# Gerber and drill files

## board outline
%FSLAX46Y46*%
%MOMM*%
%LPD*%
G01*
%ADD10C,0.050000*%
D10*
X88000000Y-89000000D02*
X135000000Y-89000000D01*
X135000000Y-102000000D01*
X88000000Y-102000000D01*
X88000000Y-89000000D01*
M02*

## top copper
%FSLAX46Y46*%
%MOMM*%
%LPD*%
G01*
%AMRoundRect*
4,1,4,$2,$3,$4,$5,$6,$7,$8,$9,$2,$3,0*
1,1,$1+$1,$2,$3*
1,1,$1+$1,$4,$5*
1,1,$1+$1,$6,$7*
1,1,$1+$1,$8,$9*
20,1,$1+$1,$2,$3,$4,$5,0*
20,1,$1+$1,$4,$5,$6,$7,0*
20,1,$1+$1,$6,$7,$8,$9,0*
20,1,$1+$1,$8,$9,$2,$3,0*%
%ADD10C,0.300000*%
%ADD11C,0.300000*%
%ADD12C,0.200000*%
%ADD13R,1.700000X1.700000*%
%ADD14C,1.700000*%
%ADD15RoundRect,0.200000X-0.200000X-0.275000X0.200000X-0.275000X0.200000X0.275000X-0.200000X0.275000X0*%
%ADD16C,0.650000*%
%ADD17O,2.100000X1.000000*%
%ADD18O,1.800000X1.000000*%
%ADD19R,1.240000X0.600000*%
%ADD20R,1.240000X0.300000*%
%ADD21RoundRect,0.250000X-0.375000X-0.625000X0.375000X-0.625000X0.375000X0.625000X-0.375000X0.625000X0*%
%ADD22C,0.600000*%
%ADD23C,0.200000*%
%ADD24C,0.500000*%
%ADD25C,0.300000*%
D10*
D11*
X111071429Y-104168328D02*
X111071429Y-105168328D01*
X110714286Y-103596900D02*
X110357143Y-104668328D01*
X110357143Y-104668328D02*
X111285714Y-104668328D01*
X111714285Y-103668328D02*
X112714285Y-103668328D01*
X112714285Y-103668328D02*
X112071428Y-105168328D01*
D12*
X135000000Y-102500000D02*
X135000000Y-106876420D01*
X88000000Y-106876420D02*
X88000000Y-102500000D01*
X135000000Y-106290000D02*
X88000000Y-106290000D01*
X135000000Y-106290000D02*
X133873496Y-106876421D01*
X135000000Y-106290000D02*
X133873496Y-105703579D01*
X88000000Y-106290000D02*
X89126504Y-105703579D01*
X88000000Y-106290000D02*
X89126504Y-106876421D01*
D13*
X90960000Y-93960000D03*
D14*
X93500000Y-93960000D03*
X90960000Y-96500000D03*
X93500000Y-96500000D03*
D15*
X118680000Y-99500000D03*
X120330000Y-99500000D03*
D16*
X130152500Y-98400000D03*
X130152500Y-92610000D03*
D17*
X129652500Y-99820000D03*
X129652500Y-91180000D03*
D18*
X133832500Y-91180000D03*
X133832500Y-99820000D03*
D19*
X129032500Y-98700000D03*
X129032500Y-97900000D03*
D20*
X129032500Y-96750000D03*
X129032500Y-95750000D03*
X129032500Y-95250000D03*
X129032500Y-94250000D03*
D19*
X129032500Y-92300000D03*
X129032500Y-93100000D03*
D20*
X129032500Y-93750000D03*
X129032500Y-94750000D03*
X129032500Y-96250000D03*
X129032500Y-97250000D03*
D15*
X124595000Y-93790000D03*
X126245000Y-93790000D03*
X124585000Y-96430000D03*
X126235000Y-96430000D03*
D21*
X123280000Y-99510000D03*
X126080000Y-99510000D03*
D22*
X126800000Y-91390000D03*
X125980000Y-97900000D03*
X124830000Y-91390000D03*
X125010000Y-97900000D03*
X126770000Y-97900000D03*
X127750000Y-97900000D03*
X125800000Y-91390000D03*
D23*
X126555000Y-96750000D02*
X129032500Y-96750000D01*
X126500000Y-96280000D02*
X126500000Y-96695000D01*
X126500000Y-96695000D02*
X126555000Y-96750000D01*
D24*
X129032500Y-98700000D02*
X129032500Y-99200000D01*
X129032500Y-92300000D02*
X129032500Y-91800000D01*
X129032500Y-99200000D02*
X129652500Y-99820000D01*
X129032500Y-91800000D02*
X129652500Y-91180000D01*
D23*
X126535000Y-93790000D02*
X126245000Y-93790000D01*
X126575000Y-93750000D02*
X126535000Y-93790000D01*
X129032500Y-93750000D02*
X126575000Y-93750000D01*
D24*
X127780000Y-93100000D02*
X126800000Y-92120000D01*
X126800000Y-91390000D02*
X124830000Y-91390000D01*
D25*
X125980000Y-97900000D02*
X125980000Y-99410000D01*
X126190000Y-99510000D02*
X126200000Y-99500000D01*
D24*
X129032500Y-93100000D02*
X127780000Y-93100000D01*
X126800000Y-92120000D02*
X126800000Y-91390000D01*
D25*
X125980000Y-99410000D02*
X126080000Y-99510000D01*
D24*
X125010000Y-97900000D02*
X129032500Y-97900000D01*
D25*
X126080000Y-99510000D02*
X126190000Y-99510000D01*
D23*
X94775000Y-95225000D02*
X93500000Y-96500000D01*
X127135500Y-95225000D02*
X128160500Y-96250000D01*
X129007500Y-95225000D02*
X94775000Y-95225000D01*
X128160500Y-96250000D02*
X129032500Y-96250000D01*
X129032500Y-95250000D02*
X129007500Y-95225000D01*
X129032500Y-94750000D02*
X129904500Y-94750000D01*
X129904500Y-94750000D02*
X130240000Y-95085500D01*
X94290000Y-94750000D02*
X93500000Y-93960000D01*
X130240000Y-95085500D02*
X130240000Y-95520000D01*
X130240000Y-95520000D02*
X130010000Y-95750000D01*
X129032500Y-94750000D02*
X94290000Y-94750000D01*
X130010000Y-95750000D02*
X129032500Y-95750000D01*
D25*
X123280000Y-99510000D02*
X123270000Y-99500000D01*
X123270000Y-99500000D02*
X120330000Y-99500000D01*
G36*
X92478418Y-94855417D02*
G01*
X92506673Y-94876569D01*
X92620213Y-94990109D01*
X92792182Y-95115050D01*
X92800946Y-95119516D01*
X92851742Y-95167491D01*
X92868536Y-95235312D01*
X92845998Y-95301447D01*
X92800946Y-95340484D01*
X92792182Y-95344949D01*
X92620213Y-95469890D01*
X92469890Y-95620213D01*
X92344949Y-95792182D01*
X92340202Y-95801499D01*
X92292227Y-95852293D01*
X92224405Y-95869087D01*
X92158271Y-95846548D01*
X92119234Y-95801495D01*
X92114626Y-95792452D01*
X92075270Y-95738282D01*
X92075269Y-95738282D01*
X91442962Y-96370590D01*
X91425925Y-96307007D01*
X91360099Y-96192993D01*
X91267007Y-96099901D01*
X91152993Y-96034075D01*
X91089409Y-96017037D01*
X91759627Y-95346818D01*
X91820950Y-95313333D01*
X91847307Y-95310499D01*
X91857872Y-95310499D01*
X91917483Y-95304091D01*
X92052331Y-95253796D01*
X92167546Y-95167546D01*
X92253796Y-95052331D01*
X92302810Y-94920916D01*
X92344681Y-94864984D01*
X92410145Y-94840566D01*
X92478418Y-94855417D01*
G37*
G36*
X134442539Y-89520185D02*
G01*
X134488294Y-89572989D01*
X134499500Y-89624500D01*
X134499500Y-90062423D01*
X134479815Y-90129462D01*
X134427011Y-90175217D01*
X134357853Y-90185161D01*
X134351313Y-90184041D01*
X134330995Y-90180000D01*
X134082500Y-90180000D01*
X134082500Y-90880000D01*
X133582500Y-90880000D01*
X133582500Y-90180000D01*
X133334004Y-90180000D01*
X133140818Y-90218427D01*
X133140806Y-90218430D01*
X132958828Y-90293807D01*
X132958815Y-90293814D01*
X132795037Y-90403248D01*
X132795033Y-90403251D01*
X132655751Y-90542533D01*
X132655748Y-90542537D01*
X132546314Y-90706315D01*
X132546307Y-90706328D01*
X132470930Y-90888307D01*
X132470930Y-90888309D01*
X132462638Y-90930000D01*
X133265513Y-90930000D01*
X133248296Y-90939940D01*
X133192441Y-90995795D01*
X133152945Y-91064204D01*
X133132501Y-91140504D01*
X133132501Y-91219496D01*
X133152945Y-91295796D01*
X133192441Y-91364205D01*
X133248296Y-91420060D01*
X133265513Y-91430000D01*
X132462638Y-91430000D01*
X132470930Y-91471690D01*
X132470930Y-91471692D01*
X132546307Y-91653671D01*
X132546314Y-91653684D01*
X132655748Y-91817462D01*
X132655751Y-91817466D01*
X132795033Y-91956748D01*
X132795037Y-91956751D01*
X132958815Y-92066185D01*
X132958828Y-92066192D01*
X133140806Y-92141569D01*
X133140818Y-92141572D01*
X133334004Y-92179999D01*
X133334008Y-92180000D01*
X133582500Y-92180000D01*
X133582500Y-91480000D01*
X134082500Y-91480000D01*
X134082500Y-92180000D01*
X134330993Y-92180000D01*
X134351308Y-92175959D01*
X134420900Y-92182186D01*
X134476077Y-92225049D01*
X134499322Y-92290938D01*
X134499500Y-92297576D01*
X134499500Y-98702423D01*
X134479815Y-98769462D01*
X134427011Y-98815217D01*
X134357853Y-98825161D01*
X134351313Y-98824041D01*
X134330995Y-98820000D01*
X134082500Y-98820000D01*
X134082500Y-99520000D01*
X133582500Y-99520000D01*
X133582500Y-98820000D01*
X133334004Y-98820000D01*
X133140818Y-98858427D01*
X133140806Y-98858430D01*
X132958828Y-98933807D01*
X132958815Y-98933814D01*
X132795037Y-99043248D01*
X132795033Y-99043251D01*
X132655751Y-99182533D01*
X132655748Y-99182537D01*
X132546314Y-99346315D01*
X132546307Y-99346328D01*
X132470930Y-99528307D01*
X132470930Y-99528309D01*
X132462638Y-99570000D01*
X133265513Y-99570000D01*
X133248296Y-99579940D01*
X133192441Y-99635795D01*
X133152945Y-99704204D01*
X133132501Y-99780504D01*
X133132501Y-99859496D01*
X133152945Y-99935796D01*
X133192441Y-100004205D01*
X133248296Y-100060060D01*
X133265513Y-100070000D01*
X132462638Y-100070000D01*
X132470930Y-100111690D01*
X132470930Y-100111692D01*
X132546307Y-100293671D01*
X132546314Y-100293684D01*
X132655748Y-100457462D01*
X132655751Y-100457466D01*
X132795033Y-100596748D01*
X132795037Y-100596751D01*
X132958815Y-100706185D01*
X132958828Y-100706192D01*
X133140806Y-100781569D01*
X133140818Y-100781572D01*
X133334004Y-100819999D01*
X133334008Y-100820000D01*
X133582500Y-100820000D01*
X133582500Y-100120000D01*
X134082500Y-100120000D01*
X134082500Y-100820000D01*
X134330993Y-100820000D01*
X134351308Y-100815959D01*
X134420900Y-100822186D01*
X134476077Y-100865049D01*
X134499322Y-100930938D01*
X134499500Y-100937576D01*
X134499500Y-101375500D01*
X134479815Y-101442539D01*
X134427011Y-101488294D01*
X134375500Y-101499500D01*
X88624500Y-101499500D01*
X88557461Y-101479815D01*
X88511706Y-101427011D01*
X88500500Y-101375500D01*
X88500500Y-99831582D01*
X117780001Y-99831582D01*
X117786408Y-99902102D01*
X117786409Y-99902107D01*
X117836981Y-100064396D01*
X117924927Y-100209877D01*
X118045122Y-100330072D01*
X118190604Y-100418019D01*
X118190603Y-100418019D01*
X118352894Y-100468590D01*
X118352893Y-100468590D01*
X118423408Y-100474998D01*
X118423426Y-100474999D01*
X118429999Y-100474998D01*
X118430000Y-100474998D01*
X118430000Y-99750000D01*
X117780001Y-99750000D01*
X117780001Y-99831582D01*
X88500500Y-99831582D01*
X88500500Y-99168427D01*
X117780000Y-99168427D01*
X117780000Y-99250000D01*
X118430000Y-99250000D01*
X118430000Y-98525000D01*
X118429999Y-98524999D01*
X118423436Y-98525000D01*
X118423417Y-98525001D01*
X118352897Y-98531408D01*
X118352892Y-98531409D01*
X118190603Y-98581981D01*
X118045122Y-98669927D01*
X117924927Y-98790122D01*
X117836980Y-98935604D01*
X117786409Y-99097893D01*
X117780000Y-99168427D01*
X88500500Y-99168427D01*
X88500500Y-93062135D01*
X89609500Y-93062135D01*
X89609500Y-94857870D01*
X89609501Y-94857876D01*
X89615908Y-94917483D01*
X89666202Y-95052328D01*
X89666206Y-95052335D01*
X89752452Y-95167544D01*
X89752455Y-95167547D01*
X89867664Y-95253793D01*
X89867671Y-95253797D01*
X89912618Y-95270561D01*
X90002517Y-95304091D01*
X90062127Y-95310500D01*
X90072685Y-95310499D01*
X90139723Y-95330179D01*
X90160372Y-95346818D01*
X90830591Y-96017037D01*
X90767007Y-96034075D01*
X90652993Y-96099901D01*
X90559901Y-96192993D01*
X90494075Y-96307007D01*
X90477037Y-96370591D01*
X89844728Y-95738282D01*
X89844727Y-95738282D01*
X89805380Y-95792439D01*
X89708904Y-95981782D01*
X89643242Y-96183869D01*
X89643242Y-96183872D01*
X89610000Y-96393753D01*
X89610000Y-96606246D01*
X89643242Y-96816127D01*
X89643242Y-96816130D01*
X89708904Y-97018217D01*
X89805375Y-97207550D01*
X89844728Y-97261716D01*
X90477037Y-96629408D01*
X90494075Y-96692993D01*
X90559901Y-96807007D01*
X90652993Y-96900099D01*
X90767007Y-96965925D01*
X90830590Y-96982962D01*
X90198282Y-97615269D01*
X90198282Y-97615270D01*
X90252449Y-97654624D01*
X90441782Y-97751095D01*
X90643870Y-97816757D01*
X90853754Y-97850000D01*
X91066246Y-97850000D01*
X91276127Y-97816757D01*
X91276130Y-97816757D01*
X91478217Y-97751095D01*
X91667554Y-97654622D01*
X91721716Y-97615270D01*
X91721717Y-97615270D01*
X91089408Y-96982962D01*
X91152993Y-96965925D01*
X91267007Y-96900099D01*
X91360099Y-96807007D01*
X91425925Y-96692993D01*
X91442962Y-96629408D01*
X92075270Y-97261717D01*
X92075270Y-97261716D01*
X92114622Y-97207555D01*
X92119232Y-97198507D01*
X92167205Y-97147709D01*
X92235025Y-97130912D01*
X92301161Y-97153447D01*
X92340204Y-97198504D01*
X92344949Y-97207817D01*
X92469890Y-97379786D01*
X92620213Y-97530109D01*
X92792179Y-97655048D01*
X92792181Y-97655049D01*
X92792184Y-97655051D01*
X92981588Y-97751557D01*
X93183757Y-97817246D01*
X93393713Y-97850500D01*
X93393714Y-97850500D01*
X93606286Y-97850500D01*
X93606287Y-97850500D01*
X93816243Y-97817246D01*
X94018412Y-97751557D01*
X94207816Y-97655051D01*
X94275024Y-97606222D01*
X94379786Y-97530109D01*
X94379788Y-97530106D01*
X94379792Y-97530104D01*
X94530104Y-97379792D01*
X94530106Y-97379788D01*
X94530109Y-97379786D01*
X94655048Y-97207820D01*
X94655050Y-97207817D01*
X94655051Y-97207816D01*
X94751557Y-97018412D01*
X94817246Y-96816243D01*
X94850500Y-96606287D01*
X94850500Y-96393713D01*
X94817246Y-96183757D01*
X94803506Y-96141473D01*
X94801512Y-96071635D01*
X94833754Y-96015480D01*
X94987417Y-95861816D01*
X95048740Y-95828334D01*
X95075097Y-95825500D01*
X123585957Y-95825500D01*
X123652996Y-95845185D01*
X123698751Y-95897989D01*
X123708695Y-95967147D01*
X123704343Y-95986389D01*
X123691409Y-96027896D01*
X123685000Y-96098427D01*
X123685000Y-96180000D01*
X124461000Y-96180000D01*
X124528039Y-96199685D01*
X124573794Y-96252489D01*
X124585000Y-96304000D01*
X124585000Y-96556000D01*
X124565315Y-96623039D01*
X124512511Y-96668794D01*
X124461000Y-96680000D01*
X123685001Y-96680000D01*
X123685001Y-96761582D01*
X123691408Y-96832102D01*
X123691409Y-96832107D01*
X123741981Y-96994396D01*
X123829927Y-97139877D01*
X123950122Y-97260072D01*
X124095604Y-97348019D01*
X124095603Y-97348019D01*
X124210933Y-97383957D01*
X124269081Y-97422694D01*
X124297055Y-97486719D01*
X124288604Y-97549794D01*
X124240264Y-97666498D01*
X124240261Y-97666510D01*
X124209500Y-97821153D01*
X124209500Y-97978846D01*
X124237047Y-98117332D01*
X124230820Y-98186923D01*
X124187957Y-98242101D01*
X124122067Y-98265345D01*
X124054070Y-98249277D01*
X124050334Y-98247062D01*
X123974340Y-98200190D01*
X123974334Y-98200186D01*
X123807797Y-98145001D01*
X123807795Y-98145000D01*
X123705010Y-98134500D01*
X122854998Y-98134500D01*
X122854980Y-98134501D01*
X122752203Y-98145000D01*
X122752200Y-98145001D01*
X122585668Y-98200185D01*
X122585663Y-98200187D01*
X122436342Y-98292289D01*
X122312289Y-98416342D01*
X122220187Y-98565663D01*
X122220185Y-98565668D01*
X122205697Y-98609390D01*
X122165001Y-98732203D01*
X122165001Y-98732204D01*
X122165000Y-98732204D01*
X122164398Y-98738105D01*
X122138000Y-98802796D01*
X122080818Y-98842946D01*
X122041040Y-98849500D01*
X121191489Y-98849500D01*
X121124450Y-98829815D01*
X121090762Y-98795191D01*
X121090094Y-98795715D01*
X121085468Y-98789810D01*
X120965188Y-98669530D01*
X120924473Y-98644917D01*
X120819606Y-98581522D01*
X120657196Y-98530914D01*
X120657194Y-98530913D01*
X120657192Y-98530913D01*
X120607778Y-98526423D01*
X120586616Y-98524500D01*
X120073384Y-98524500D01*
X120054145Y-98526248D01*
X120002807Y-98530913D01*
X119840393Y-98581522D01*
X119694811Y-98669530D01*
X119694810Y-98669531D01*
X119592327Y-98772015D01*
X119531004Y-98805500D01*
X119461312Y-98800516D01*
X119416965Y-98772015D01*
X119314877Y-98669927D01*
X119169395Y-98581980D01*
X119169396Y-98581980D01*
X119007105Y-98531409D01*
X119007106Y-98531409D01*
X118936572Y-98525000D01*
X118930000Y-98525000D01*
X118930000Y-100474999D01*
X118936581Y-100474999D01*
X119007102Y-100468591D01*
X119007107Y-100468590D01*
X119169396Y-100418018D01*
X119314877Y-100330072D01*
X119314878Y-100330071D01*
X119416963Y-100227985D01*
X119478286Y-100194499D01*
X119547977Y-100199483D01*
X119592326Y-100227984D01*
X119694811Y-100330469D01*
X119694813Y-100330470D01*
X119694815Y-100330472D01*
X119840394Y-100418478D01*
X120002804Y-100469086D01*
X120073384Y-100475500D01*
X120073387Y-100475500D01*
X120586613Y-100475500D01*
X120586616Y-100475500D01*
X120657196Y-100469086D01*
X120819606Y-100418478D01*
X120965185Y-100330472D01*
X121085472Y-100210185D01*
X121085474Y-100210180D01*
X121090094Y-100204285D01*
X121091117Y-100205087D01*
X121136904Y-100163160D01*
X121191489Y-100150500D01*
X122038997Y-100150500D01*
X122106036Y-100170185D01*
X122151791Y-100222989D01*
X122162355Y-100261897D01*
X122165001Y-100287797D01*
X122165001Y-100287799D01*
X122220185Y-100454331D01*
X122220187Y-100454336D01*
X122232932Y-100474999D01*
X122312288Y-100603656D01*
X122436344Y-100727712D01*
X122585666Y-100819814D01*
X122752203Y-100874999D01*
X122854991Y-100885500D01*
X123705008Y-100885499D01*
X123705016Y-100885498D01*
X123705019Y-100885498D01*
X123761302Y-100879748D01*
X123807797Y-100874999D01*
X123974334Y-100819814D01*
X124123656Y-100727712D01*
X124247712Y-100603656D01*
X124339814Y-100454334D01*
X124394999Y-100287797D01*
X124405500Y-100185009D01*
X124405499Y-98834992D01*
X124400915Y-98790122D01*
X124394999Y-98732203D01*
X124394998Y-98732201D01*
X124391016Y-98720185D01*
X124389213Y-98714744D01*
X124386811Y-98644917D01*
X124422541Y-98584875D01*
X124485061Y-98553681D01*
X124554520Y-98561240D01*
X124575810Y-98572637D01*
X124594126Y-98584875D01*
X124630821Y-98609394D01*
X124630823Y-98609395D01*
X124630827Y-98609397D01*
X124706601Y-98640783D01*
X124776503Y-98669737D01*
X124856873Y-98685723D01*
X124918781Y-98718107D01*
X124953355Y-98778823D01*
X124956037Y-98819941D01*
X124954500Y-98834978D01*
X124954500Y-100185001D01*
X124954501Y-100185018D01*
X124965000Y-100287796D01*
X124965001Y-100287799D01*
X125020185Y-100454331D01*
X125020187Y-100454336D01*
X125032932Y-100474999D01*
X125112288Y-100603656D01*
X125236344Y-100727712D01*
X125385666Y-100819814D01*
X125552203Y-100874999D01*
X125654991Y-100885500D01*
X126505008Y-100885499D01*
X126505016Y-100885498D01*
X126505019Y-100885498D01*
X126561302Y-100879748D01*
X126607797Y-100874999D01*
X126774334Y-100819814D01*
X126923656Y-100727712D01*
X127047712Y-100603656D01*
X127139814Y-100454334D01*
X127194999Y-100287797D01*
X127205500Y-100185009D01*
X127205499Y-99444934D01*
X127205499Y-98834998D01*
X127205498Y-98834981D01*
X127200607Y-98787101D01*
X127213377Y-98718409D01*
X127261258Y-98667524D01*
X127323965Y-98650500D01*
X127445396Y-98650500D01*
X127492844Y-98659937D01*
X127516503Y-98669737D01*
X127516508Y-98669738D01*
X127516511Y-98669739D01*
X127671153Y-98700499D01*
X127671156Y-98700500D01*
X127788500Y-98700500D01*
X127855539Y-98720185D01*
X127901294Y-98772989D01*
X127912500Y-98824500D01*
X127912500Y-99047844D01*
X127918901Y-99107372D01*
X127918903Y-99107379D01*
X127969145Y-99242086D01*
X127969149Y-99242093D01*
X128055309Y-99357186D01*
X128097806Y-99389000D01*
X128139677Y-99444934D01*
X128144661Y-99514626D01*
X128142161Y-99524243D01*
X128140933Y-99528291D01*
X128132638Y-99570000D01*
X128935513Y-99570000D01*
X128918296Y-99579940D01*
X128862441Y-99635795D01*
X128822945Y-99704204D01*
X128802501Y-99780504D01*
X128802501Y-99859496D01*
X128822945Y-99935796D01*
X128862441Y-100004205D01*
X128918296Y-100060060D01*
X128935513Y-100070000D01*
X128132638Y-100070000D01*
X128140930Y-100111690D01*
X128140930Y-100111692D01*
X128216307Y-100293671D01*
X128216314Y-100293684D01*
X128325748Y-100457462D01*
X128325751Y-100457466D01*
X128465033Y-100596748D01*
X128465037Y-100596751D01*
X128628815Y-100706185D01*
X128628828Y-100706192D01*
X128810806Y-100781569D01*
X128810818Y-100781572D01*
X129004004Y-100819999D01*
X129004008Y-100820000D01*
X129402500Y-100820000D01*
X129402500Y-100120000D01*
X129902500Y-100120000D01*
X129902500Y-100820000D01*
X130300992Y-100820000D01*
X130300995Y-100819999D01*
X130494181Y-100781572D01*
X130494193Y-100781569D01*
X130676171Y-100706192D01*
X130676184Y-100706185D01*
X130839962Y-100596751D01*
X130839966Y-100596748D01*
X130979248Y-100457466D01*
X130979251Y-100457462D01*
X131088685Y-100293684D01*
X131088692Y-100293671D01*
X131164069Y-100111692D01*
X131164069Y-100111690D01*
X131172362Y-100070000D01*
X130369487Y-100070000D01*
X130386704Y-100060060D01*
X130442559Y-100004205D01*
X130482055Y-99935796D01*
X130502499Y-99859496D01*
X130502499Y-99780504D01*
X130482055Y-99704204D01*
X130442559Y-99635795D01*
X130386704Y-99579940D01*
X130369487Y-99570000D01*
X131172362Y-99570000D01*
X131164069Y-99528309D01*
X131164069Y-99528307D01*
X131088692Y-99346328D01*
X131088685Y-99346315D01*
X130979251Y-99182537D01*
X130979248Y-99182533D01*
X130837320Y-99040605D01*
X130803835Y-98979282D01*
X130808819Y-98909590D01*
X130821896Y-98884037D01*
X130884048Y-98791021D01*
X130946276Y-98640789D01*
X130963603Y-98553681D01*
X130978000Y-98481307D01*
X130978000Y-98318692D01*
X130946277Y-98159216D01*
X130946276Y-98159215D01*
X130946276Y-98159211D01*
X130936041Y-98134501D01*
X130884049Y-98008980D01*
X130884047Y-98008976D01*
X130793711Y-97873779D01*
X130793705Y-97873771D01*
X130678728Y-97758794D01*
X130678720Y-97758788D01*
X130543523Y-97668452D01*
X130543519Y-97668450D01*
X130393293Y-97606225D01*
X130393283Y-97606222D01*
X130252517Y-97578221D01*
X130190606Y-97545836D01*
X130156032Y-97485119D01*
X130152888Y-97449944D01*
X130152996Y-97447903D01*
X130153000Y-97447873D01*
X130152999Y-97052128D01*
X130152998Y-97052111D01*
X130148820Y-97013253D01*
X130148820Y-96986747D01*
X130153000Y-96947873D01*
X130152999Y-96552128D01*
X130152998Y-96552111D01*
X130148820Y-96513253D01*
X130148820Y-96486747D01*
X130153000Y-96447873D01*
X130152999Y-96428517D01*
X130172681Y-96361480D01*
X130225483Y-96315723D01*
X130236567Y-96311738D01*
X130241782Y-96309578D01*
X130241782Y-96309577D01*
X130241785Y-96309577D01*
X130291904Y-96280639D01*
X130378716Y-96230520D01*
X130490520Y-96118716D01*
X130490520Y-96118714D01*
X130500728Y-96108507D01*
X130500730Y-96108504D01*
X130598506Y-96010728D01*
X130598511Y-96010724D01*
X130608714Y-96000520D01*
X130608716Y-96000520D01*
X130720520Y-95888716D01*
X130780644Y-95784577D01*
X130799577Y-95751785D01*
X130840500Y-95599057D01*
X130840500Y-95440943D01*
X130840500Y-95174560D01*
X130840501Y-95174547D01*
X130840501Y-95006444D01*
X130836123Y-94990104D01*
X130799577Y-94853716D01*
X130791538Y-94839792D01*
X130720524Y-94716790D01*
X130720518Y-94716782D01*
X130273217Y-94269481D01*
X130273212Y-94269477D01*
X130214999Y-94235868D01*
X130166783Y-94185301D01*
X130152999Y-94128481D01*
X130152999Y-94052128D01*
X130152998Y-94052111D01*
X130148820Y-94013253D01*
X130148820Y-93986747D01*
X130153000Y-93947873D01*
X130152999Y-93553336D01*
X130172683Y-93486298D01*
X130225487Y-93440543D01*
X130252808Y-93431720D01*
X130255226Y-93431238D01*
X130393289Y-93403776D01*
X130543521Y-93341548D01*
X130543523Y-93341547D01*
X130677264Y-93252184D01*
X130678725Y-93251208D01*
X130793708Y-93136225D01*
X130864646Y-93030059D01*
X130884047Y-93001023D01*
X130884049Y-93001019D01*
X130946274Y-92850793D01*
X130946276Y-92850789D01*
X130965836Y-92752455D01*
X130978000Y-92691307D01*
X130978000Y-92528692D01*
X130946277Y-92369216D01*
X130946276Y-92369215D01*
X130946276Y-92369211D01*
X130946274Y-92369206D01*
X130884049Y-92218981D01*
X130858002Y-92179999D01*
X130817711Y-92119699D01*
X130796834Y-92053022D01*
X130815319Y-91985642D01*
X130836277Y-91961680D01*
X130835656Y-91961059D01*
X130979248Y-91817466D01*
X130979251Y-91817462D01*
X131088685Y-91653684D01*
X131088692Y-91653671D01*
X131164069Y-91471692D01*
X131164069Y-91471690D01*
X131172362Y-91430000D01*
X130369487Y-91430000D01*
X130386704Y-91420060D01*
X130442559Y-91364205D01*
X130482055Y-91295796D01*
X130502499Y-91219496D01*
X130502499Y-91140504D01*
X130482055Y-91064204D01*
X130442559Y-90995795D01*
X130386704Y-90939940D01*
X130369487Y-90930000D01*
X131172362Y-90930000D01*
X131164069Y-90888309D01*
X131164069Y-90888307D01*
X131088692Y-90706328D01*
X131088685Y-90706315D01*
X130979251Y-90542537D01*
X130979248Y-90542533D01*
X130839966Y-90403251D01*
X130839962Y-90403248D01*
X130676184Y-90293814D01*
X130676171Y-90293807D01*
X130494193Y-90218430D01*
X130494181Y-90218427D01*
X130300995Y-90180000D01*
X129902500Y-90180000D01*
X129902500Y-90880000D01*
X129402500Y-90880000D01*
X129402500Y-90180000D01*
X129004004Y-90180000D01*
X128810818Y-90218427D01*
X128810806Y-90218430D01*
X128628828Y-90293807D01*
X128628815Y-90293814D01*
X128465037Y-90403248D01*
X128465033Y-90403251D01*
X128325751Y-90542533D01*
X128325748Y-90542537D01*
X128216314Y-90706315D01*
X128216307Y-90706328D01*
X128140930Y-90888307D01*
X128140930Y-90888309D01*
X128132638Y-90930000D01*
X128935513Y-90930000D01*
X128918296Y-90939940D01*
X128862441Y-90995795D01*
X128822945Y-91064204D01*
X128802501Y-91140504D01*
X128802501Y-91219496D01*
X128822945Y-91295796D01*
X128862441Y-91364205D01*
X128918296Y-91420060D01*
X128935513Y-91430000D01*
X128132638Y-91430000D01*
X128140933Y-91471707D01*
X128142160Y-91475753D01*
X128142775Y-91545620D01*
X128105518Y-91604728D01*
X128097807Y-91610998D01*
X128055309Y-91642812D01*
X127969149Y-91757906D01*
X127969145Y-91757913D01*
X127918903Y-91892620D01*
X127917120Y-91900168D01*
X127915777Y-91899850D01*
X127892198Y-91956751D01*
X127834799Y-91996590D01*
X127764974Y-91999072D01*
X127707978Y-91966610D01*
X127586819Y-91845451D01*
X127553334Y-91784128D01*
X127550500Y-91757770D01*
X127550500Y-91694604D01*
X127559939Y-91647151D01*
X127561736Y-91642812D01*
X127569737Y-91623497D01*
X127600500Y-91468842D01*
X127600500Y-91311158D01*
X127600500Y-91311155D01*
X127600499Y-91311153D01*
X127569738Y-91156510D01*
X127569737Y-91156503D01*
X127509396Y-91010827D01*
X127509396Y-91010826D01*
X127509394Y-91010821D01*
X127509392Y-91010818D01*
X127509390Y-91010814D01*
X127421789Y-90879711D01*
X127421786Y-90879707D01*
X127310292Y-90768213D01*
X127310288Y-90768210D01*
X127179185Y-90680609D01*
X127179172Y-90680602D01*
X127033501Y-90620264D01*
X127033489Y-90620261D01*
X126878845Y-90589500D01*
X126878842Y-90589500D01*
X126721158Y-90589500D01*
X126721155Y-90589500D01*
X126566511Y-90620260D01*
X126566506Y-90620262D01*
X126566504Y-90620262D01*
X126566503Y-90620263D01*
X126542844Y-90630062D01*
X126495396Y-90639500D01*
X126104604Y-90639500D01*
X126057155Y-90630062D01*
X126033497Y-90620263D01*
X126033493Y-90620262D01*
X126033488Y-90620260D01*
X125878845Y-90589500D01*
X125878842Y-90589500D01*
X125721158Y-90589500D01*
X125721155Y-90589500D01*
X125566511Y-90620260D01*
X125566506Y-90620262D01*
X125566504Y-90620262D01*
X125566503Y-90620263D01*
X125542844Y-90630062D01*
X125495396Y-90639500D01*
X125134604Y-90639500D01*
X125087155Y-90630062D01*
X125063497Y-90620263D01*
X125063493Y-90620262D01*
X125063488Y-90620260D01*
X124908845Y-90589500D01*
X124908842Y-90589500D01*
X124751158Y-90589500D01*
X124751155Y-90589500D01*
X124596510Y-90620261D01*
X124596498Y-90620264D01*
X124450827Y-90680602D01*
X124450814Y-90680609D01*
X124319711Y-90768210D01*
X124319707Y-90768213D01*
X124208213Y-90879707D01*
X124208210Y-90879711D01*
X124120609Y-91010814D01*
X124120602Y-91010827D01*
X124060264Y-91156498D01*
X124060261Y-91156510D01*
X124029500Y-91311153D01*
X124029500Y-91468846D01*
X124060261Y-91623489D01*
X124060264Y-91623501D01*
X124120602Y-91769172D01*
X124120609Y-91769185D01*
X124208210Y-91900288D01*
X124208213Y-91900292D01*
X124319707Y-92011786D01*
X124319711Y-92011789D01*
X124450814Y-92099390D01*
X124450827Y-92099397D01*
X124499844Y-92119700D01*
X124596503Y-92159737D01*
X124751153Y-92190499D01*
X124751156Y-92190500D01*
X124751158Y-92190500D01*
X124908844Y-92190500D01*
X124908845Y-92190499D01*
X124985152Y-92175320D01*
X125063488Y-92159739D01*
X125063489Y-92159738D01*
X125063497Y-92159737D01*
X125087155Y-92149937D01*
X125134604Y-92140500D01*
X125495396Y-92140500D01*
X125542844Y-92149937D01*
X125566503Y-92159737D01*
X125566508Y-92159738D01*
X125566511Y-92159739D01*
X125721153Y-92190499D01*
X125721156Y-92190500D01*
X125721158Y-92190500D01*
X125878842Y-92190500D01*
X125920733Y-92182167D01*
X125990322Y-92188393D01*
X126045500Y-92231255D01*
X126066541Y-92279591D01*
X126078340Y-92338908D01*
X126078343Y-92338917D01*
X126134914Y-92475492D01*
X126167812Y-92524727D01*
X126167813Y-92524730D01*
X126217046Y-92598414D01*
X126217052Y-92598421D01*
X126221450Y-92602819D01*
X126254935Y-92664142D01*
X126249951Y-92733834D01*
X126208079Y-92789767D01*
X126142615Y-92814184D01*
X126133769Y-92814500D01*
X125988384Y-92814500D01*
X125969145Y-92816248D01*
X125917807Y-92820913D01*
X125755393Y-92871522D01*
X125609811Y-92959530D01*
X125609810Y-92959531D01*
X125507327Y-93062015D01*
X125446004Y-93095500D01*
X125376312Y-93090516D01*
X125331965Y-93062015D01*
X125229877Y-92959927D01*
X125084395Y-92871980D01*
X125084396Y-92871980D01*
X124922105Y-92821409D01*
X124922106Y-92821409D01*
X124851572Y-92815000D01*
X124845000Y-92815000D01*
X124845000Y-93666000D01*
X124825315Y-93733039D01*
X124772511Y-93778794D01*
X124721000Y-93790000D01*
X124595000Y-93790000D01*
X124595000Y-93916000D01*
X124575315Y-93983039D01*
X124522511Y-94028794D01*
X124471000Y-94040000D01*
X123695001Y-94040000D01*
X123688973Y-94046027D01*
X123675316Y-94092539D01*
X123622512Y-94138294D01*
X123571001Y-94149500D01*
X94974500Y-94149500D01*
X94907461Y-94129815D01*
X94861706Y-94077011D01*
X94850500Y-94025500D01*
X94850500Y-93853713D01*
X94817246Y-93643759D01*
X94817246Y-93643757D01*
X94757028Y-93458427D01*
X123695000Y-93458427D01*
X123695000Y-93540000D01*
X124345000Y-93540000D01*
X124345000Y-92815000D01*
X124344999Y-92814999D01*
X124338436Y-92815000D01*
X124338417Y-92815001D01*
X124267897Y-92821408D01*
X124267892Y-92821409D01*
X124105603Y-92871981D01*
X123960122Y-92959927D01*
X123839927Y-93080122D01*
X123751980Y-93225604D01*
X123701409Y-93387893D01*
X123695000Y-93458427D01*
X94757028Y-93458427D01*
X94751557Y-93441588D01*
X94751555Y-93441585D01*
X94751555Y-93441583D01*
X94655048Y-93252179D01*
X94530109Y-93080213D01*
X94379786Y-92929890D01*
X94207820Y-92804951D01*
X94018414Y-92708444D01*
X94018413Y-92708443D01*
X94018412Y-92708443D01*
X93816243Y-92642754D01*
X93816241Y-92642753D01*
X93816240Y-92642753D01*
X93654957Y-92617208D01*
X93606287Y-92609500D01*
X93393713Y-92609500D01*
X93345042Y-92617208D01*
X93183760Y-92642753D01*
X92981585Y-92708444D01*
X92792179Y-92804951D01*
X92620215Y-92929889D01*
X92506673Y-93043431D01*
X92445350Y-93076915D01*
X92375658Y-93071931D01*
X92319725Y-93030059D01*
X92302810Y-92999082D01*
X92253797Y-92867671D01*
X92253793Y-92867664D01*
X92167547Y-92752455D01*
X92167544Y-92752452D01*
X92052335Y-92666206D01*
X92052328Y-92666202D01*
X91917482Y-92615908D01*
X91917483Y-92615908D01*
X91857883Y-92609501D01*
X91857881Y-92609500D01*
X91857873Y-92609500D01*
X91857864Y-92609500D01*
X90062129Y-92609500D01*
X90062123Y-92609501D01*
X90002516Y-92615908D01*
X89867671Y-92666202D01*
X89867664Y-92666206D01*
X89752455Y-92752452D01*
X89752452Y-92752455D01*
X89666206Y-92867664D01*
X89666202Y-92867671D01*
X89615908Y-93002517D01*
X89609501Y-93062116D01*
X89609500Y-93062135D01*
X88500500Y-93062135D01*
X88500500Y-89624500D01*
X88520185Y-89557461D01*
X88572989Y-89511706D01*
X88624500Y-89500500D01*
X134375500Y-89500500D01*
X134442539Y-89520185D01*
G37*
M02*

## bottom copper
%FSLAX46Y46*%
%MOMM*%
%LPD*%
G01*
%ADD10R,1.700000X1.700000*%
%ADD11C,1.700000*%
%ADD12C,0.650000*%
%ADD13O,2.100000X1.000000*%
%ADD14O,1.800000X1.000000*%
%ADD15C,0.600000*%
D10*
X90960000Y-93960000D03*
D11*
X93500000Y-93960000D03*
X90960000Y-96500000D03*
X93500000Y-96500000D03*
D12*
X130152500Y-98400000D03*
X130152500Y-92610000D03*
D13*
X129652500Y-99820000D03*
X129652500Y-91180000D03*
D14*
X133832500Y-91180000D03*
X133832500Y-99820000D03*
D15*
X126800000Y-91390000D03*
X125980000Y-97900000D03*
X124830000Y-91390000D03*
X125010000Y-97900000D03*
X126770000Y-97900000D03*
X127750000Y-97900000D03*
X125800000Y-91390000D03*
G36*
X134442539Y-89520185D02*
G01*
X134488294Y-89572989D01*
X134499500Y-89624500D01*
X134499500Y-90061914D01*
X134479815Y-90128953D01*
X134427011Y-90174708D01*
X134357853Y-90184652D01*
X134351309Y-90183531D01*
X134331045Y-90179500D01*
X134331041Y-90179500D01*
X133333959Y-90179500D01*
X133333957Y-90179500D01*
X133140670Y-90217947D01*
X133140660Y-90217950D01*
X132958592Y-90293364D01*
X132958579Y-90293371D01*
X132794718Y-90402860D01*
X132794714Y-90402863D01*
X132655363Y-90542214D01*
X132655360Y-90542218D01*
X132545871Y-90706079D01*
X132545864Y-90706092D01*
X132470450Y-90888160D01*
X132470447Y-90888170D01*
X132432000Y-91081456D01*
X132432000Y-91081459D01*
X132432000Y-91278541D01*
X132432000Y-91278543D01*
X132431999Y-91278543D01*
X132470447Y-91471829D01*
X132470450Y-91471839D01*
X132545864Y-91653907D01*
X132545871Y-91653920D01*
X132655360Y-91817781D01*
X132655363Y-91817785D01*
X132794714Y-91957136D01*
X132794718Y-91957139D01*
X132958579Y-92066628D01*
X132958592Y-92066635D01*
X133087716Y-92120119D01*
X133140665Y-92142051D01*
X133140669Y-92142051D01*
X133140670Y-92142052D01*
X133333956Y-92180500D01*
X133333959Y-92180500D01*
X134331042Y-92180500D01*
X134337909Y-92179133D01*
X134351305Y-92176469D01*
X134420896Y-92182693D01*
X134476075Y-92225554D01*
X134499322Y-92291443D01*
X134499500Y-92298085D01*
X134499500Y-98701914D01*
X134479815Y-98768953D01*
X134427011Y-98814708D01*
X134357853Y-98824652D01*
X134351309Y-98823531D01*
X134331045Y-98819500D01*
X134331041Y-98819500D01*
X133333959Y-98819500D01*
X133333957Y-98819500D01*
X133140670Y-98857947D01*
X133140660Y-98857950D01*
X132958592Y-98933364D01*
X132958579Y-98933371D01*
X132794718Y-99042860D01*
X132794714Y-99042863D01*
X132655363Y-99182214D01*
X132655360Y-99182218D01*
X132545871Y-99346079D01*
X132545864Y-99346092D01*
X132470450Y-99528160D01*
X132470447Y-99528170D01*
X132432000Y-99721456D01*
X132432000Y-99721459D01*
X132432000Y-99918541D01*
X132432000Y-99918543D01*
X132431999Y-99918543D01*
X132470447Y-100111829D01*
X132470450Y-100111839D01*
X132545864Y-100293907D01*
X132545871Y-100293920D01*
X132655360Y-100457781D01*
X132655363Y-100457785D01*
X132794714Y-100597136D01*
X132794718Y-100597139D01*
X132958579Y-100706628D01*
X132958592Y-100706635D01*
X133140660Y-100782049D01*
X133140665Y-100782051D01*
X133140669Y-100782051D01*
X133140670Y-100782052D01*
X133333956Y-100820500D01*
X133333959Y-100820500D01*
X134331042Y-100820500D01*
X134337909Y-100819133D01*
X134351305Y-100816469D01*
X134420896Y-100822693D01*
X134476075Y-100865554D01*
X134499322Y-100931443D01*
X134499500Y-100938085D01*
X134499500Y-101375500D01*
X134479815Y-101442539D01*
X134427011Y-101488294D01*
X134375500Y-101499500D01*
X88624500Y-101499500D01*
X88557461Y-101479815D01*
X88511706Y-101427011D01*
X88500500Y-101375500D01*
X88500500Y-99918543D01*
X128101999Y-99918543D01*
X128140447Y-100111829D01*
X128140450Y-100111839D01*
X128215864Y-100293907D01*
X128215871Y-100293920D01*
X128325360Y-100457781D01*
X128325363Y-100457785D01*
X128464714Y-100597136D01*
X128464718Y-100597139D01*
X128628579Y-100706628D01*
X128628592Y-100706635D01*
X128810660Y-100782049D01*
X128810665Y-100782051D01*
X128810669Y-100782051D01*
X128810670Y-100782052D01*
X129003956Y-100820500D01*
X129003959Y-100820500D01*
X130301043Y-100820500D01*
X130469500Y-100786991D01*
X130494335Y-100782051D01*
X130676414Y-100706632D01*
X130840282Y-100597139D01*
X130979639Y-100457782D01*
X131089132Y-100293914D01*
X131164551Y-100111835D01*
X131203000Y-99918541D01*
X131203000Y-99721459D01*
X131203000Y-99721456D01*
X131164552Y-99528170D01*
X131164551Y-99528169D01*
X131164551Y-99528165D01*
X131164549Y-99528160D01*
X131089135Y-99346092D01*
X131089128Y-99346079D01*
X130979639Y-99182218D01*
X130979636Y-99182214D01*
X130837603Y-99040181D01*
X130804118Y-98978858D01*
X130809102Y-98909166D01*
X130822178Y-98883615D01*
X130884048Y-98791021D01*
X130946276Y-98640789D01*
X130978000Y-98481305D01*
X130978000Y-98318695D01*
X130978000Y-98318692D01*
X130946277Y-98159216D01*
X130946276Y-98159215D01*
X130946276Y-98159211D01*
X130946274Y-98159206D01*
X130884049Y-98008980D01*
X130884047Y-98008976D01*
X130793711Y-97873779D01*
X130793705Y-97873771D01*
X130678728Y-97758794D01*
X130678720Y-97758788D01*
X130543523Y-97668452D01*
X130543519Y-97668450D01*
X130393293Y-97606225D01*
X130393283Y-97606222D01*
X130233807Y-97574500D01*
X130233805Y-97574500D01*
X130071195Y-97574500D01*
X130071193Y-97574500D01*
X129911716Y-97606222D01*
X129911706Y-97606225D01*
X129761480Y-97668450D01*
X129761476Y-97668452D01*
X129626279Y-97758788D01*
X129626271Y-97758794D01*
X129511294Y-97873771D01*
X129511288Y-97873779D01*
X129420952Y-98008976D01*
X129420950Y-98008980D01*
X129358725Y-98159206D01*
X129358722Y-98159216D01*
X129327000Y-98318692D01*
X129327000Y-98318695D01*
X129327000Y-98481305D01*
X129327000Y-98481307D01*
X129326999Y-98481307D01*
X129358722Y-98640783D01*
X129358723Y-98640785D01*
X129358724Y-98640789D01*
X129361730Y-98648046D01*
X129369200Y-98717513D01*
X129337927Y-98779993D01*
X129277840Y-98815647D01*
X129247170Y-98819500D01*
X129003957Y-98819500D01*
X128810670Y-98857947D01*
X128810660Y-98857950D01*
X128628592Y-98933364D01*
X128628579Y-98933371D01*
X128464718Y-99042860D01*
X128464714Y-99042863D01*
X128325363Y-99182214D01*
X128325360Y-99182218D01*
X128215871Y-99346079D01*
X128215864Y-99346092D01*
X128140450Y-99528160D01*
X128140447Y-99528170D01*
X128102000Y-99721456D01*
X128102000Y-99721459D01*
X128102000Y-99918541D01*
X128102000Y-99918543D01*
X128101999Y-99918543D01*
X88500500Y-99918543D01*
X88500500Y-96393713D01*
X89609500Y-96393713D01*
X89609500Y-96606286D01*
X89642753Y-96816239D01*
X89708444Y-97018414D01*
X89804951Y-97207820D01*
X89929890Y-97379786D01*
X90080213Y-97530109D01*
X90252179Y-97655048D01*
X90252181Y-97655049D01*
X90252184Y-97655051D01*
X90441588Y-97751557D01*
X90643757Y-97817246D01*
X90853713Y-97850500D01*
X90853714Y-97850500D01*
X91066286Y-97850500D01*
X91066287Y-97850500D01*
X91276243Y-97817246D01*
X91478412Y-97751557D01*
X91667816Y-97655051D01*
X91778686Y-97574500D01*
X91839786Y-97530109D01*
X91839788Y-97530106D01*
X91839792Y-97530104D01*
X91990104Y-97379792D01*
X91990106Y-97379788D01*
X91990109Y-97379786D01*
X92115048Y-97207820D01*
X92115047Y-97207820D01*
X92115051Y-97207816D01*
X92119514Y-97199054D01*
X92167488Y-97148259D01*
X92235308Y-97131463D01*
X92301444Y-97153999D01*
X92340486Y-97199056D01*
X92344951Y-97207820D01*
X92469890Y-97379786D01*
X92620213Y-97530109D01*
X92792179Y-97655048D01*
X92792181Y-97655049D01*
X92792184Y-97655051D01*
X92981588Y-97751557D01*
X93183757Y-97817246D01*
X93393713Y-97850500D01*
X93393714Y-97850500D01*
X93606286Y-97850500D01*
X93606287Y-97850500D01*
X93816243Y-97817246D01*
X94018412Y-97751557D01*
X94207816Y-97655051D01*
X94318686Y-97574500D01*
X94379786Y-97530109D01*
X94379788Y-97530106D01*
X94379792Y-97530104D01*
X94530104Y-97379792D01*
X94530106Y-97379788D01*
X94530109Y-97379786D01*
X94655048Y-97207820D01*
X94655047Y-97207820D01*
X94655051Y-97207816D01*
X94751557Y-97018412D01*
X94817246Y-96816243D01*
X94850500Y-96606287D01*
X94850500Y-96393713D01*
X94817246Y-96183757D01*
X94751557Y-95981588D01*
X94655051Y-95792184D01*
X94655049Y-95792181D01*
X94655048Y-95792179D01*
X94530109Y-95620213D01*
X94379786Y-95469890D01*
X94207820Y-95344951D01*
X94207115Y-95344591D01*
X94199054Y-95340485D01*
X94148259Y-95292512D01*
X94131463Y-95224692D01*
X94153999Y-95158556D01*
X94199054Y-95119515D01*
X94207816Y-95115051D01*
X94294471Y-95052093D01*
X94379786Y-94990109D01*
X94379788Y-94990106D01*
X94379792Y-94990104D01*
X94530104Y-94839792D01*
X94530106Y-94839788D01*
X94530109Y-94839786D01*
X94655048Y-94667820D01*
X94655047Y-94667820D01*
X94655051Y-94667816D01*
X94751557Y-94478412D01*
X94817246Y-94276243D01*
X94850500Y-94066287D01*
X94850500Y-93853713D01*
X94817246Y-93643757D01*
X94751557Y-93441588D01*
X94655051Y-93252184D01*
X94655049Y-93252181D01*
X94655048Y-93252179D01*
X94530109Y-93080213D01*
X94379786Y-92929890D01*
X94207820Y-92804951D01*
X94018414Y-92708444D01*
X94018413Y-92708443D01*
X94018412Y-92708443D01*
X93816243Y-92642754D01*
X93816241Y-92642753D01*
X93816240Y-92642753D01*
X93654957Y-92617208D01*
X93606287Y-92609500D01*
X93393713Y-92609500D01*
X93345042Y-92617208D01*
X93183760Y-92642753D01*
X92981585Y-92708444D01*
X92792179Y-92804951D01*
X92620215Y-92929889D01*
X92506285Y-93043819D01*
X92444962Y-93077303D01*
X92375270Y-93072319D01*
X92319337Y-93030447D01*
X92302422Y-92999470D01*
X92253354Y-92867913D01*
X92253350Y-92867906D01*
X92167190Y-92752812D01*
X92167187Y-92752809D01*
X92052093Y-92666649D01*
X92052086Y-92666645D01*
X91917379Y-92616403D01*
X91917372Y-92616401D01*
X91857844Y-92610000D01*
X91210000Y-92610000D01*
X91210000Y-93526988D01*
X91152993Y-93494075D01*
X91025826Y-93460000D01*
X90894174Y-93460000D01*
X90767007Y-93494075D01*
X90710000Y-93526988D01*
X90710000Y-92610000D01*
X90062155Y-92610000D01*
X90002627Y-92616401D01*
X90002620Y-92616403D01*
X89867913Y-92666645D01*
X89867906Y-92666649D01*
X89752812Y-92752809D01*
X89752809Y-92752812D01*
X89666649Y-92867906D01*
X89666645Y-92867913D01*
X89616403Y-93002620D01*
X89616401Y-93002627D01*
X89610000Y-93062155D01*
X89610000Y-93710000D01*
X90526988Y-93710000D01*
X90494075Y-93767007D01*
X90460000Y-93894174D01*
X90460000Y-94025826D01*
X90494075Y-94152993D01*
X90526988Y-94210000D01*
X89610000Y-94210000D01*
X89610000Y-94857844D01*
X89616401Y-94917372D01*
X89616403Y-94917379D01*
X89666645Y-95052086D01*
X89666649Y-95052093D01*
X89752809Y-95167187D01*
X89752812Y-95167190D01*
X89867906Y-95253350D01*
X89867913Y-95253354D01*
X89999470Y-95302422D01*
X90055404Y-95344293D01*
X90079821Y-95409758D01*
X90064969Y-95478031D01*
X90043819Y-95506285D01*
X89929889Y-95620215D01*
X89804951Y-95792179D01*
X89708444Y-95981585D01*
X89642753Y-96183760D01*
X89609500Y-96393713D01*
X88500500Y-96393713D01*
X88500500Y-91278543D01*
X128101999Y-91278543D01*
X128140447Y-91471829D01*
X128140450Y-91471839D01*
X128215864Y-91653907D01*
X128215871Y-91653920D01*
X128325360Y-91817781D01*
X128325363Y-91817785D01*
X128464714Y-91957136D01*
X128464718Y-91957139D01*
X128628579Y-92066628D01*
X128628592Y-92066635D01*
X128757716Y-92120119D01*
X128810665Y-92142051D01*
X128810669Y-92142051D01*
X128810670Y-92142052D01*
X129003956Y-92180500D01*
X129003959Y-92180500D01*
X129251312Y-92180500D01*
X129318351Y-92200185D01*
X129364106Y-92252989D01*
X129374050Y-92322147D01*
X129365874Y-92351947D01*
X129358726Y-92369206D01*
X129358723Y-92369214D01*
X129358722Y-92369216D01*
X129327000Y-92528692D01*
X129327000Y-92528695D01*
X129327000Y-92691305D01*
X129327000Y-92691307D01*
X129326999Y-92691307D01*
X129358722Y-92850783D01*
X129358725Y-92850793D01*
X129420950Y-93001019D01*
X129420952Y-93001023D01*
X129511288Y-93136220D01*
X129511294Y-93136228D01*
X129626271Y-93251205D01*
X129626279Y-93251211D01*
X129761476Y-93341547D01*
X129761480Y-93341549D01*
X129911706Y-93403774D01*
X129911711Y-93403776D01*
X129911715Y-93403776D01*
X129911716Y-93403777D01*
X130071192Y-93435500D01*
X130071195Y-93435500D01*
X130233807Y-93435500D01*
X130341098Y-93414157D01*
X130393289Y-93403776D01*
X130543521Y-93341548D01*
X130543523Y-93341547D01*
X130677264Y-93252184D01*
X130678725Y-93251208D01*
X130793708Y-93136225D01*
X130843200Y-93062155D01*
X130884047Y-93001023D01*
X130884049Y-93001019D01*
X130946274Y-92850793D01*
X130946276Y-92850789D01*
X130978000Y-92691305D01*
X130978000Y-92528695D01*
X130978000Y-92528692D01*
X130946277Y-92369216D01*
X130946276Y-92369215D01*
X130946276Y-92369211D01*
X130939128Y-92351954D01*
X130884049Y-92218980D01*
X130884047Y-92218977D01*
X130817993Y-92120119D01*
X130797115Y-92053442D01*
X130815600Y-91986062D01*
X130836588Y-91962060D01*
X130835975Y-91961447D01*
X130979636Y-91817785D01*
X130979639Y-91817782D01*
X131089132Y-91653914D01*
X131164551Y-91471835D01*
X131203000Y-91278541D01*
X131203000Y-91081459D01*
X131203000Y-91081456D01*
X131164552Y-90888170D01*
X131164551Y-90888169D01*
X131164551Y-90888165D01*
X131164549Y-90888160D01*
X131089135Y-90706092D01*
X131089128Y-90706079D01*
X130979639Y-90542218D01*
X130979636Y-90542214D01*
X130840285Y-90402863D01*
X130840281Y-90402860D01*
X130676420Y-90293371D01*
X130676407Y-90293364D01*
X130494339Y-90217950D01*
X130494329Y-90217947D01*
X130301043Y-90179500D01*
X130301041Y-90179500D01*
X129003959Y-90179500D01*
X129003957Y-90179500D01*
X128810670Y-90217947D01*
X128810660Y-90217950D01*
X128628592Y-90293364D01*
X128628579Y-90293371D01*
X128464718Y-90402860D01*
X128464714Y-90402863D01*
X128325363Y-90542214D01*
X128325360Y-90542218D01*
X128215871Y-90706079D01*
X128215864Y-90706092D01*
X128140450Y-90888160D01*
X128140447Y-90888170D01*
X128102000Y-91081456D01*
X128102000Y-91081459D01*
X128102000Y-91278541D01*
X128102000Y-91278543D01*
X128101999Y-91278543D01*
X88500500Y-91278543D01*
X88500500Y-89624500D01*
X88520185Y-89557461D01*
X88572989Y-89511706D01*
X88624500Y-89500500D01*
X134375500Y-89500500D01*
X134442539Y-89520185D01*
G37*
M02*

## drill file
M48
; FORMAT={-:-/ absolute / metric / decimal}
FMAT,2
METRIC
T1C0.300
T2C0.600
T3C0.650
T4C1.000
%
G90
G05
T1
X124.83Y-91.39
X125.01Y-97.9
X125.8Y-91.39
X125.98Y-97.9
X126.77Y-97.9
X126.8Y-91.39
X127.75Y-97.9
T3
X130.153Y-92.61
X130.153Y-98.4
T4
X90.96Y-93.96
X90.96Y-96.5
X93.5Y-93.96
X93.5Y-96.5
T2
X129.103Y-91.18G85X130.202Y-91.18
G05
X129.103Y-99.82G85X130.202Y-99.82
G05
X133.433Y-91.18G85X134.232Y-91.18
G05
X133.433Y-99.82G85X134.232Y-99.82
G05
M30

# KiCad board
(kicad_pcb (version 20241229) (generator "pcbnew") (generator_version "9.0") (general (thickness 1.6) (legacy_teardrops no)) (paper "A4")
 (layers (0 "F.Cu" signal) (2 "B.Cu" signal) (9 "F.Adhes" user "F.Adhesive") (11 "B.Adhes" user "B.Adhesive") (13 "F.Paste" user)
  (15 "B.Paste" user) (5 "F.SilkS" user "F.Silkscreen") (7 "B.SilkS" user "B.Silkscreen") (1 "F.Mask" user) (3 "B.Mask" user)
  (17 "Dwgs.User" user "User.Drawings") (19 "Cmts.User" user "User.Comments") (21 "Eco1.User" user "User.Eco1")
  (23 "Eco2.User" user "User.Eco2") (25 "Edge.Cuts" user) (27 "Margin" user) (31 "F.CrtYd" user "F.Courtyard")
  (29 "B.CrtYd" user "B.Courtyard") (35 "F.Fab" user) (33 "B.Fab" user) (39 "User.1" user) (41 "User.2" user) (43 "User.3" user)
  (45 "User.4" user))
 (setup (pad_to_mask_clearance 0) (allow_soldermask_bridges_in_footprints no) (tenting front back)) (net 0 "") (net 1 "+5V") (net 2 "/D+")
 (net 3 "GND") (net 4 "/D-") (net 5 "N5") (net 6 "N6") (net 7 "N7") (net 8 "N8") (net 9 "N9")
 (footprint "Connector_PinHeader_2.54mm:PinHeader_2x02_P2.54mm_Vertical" (layer "F.Cu") (at 90.96 93.96)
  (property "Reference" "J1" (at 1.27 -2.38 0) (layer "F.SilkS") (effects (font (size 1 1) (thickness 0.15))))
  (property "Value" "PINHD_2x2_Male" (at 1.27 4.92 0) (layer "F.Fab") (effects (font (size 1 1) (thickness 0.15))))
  (pad "1" thru_hole rect (at 0 0) (size 1.7 1.7) (drill 1) (layers "*.Cu" "*.Mask") (remove_unused_layers no) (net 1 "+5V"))
  (pad "2" thru_hole circle (at 2.54 0) (size 1.7 1.7) (drill 1) (layers "*.Cu" "*.Mask") (remove_unused_layers no) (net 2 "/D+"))
  (pad "3" thru_hole circle (at 0 2.54) (size 1.7 1.7) (drill 1) (layers "*.Cu" "*.Mask") (remove_unused_layers no) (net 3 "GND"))
  (pad "4" thru_hole circle (at 2.54 2.54) (size 1.7 1.7) (drill 1) (layers "*.Cu" "*.Mask") (remove_unused_layers no) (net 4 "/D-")))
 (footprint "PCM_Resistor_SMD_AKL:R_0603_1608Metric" (layer "F.Cu") (at 119.505 99.5)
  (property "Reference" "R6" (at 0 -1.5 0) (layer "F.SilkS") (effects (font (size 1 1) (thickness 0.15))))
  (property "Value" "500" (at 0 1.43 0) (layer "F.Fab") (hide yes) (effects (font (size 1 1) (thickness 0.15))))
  (pad "1" smd roundrect (at -0.825 0) (size 0.8 0.95) (layers "F.Cu" "F.Mask" "F.Paste") (roundrect_rratio 0.25) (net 3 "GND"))
  (pad "2" smd roundrect (at 0.825 0) (size 0.8 0.95) (layers "F.Cu" "F.Mask" "F.Paste") (roundrect_rratio 0.25) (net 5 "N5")))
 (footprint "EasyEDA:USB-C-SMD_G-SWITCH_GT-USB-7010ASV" (layer "F.Cu") (at 131.4325 95.5 90)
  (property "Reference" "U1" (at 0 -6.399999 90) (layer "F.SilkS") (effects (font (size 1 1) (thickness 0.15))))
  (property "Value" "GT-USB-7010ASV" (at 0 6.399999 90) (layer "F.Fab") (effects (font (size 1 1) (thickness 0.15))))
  (pad "" thru_hole circle (at -2.9 -1.28 90) (size 0.65 0.65) (drill 0.65) (layers "*.Cu" "*.Mask") (remove_unused_layers no))
  (pad "" thru_hole circle (at 2.89 -1.28 90) (size 0.65 0.65) (drill 0.65) (layers "*.Cu" "*.Mask") (remove_unused_layers no))
  (pad "1" thru_hole oval (at -4.32 -1.78 90) (size 1 2.1) (drill oval 0.599999 1.699997) (layers "*.Cu" "*.Mask") (remove_unused_layers no)
   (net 3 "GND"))
  (pad "2" thru_hole oval (at 4.32 -1.78 90) (size 1 2.1) (drill oval 0.599999 1.699997) (layers "*.Cu" "*.Mask") (remove_unused_layers no)
   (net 3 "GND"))
  (pad "3" thru_hole oval (at 4.32 2.4 90) (size 1 1.8) (drill oval 0.599999 1.399997) (layers "*.Cu" "*.Mask") (remove_unused_layers no)
   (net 3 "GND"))
  (pad "4" thru_hole oval (at -4.32 2.4 90) (size 1 1.8) (drill oval 0.599999 1.399997) (layers "*.Cu" "*.Mask") (remove_unused_layers no)
   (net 3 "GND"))
  (pad "A1B12" smd rect (at -3.2 -2.4 90) (size 0.6 1.24) (layers "F.Cu" "F.Mask" "F.Paste") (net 3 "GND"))
  (pad "A4B9" smd rect (at -2.4 -2.4 90) (size 0.6 1.24) (layers "F.Cu" "F.Mask" "F.Paste") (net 1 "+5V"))
  (pad "A5" smd rect (at -1.25 -2.4 90) (size 0.3 1.24) (layers "F.Cu" "F.Mask" "F.Paste") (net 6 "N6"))
  (pad "A6" smd rect (at -0.25 -2.4 90) (size 0.3 1.24) (layers "F.Cu" "F.Mask" "F.Paste") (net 2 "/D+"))
  (pad "A7" smd rect (at 0.25 -2.4 90) (size 0.3 1.24) (layers "F.Cu" "F.Mask" "F.Paste") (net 4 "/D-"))
  (pad "A8" smd rect (at 1.25 -2.4 90) (size 0.3 1.24) (layers "F.Cu" "F.Mask" "F.Paste") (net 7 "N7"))
  (pad "B1A12" smd rect (at 3.2 -2.4 90) (size 0.6 1.24) (layers "F.Cu" "F.Mask" "F.Paste") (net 3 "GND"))
  (pad "B4A9" smd rect (at 2.4 -2.4 90) (size 0.6 1.24) (layers "F.Cu" "F.Mask" "F.Paste") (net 1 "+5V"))
  (pad "B5" smd rect (at 1.75 -2.4 90) (size 0.3 1.24) (layers "F.Cu" "F.Mask" "F.Paste") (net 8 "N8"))
  (pad "B6" smd rect (at 0.75 -2.4 90) (size 0.3 1.24) (layers "F.Cu" "F.Mask" "F.Paste") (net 2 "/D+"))
  (pad "B7" smd rect (at -0.75 -2.4 90) (size 0.3 1.24) (layers "F.Cu" "F.Mask" "F.Paste") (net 4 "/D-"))
  (pad "B8" smd rect (at -1.75 -2.4 90) (size 0.3 1.24) (layers "F.Cu" "F.Mask" "F.Paste") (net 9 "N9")))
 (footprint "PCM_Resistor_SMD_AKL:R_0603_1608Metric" (layer "F.Cu") (at 125.42 93.79)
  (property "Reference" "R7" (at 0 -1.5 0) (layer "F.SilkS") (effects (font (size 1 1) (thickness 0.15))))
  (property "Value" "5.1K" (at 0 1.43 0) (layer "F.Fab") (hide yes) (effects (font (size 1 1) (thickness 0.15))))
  (pad "1" smd roundrect (at -0.825 0) (size 0.8 0.95) (layers "F.Cu" "F.Mask" "F.Paste") (roundrect_rratio 0.25) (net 3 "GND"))
  (pad "2" smd roundrect (at 0.825 0) (size 0.8 0.95) (layers "F.Cu" "F.Mask" "F.Paste") (roundrect_rratio 0.25) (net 8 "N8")))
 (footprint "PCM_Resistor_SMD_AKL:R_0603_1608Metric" (layer "F.Cu") (at 125.41 96.43)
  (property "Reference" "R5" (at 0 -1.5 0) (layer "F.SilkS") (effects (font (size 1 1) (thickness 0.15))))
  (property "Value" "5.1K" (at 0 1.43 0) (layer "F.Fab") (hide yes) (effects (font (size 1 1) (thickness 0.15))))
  (pad "1" smd roundrect (at -0.825 0) (size 0.8 0.95) (layers "F.Cu" "F.Mask" "F.Paste") (roundrect_rratio 0.25) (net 3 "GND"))
  (pad "2" smd roundrect (at 0.825 0) (size 0.8 0.95) (layers "F.Cu" "F.Mask" "F.Paste") (roundrect_rratio 0.25) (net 6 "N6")))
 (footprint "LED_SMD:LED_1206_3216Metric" (layer "F.Cu") (at 124.68 99.51)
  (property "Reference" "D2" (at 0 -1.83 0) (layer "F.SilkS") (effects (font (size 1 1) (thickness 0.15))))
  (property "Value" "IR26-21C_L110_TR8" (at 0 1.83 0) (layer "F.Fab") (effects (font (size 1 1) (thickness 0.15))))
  (pad "1" smd roundrect (at -1.4 0) (size 1.25 1.75) (layers "F.Cu" "F.Mask" "F.Paste") (roundrect_rratio 0.2) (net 5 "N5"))
  (pad "2" smd roundrect (at 1.4 0) (size 1.25 1.75) (layers "F.Cu" "F.Mask" "F.Paste") (roundrect_rratio 0.2) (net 1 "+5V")))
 (gr_rect (start 88 89) (end 135 102) (stroke (width 0.05) (type default)) (fill no) (layer "Edge.Cuts"))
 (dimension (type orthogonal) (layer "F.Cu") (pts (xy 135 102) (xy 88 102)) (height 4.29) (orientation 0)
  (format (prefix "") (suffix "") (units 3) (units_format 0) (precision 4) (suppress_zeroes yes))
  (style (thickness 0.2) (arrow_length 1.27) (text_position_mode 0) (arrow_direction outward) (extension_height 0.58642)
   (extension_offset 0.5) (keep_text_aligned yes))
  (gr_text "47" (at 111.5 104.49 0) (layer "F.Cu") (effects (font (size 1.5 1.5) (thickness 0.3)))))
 (segment (start 126.555 96.75) (end 129.0325 96.75) (width 0.2) (layer "F.Cu") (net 6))
 (segment (start 126.5 96.28) (end 126.5 96.695) (width 0.2) (layer "F.Cu") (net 6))
 (segment (start 126.5 96.695) (end 126.555 96.75) (width 0.2) (layer "F.Cu") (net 6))
 (segment (start 129.0325 98.7) (end 129.0325 99.2) (width 0.5) (layer "F.Cu") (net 3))
 (segment (start 129.0325 92.3) (end 129.0325 91.8) (width 0.5) (layer "F.Cu") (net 3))
 (segment (start 129.0325 99.2) (end 129.6525 99.82) (width 0.5) (layer "F.Cu") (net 3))
 (segment (start 129.0325 91.8) (end 129.6525 91.18) (width 0.5) (layer "F.Cu") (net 3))
 (segment (start 126.535 93.79) (end 126.245 93.79) (width 0.2) (layer "F.Cu") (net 8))
 (segment (start 126.575 93.75) (end 126.535 93.79) (width 0.2) (layer "F.Cu") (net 8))
 (segment (start 129.0325 93.75) (end 126.575 93.75) (width 0.2) (layer "F.Cu") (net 8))
 (segment (start 127.78 93.1) (end 126.8 92.12) (width 0.5) (layer "F.Cu") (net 1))
 (segment (start 126.8 91.39) (end 124.83 91.39) (width 0.5) (layer "F.Cu") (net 1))
 (segment (start 125.98 97.9) (end 125.98 99.41) (width 0.3) (layer "F.Cu") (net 1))
 (segment (start 126.19 99.51) (end 126.2 99.5) (width 0.3) (layer "F.Cu") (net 1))
 (segment (start 129.0325 93.1) (end 127.78 93.1) (width 0.5) (layer "F.Cu") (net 1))
 (segment (start 126.8 92.12) (end 126.8 91.39) (width 0.5) (layer "F.Cu") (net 1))
 (segment (start 125.98 99.41) (end 126.08 99.51) (width 0.3) (layer "F.Cu") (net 1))
 (segment (start 125.01 97.9) (end 129.0325 97.9) (width 0.5) (layer "F.Cu") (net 1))
 (segment (start 126.08 99.51) (end 126.19 99.51) (width 0.3) (layer "F.Cu") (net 1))
 (via (at 126.8 91.39) (size 0.6) (drill 0.3) (layers "F.Cu" "B.Cu") (free yes) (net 1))
 (via (at 125.98 97.9) (size 0.6) (drill 0.3) (layers "F.Cu" "B.Cu") (free yes) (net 1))
 (via (at 124.83 91.39) (size 0.6) (drill 0.3) (layers "F.Cu" "B.Cu") (free yes) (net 1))
 (via (at 125.01 97.9) (size 0.6) (drill 0.3) (layers "F.Cu" "B.Cu") (free yes) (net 1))
 (via (at 126.77 97.9) (size 0.6) (drill 0.3) (layers "F.Cu" "B.Cu") (free yes) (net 1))
 (via (at 127.75 97.9) (size 0.6) (drill 0.3) (layers "F.Cu" "B.Cu") (free yes) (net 1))
 (via (at 125.8 91.39) (size 0.6) (drill 0.3) (layers "F.Cu" "B.Cu") (free yes) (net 1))
 (segment (start 94.775 95.225) (end 93.5 96.5) (width 0.2) (layer "F.Cu") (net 4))
 (segment (start 127.1355 95.225) (end 128.1605 96.25) (width 0.2) (layer "F.Cu") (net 4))
 (segment (start 129.0075 95.225) (end 94.775 95.225) (width 0.2) (layer "F.Cu") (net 4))
 (segment (start 128.1605 96.25) (end 129.0325 96.25) (width 0.2) (layer "F.Cu") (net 4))
 (segment (start 129.0325 95.25) (end 129.0075 95.225) (width 0.2) (layer "F.Cu") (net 4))
 (segment (start 129.0325 94.75) (end 129.9045 94.75) (width 0.2) (layer "F.Cu") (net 2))
 (segment (start 129.9045 94.75) (end 130.24 95.0855) (width 0.2) (layer "F.Cu") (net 2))
 (segment (start 94.29 94.75) (end 93.5 93.96) (width 0.2) (layer "F.Cu") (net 2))
 (segment (start 130.24 95.0855) (end 130.24 95.52) (width 0.2) (layer "F.Cu") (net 2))
 (segment (start 130.24 95.52) (end 130.01 95.75) (width 0.2) (layer "F.Cu") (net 2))
 (segment (start 129.0325 94.75) (end 94.29 94.75) (width 0.2) (layer "F.Cu") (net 2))
 (segment (start 130.01 95.75) (end 129.0325 95.75) (width 0.2) (layer "F.Cu") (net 2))
 (segment (start 123.28 99.51) (end 123.27 99.5) (width 0.3) (layer "F.Cu") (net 5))
 (segment (start 123.27 99.5) (end 120.33 99.5) (width 0.3) (layer "F.Cu") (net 5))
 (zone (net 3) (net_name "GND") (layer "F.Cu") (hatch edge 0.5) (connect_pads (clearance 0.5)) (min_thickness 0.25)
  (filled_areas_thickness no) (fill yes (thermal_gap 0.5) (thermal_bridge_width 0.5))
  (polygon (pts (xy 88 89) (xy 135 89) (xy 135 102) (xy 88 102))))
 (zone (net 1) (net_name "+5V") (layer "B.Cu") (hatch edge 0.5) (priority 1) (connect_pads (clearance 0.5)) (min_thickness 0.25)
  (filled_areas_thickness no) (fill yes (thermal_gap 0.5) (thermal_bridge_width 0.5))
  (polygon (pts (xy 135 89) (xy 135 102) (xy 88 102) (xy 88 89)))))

